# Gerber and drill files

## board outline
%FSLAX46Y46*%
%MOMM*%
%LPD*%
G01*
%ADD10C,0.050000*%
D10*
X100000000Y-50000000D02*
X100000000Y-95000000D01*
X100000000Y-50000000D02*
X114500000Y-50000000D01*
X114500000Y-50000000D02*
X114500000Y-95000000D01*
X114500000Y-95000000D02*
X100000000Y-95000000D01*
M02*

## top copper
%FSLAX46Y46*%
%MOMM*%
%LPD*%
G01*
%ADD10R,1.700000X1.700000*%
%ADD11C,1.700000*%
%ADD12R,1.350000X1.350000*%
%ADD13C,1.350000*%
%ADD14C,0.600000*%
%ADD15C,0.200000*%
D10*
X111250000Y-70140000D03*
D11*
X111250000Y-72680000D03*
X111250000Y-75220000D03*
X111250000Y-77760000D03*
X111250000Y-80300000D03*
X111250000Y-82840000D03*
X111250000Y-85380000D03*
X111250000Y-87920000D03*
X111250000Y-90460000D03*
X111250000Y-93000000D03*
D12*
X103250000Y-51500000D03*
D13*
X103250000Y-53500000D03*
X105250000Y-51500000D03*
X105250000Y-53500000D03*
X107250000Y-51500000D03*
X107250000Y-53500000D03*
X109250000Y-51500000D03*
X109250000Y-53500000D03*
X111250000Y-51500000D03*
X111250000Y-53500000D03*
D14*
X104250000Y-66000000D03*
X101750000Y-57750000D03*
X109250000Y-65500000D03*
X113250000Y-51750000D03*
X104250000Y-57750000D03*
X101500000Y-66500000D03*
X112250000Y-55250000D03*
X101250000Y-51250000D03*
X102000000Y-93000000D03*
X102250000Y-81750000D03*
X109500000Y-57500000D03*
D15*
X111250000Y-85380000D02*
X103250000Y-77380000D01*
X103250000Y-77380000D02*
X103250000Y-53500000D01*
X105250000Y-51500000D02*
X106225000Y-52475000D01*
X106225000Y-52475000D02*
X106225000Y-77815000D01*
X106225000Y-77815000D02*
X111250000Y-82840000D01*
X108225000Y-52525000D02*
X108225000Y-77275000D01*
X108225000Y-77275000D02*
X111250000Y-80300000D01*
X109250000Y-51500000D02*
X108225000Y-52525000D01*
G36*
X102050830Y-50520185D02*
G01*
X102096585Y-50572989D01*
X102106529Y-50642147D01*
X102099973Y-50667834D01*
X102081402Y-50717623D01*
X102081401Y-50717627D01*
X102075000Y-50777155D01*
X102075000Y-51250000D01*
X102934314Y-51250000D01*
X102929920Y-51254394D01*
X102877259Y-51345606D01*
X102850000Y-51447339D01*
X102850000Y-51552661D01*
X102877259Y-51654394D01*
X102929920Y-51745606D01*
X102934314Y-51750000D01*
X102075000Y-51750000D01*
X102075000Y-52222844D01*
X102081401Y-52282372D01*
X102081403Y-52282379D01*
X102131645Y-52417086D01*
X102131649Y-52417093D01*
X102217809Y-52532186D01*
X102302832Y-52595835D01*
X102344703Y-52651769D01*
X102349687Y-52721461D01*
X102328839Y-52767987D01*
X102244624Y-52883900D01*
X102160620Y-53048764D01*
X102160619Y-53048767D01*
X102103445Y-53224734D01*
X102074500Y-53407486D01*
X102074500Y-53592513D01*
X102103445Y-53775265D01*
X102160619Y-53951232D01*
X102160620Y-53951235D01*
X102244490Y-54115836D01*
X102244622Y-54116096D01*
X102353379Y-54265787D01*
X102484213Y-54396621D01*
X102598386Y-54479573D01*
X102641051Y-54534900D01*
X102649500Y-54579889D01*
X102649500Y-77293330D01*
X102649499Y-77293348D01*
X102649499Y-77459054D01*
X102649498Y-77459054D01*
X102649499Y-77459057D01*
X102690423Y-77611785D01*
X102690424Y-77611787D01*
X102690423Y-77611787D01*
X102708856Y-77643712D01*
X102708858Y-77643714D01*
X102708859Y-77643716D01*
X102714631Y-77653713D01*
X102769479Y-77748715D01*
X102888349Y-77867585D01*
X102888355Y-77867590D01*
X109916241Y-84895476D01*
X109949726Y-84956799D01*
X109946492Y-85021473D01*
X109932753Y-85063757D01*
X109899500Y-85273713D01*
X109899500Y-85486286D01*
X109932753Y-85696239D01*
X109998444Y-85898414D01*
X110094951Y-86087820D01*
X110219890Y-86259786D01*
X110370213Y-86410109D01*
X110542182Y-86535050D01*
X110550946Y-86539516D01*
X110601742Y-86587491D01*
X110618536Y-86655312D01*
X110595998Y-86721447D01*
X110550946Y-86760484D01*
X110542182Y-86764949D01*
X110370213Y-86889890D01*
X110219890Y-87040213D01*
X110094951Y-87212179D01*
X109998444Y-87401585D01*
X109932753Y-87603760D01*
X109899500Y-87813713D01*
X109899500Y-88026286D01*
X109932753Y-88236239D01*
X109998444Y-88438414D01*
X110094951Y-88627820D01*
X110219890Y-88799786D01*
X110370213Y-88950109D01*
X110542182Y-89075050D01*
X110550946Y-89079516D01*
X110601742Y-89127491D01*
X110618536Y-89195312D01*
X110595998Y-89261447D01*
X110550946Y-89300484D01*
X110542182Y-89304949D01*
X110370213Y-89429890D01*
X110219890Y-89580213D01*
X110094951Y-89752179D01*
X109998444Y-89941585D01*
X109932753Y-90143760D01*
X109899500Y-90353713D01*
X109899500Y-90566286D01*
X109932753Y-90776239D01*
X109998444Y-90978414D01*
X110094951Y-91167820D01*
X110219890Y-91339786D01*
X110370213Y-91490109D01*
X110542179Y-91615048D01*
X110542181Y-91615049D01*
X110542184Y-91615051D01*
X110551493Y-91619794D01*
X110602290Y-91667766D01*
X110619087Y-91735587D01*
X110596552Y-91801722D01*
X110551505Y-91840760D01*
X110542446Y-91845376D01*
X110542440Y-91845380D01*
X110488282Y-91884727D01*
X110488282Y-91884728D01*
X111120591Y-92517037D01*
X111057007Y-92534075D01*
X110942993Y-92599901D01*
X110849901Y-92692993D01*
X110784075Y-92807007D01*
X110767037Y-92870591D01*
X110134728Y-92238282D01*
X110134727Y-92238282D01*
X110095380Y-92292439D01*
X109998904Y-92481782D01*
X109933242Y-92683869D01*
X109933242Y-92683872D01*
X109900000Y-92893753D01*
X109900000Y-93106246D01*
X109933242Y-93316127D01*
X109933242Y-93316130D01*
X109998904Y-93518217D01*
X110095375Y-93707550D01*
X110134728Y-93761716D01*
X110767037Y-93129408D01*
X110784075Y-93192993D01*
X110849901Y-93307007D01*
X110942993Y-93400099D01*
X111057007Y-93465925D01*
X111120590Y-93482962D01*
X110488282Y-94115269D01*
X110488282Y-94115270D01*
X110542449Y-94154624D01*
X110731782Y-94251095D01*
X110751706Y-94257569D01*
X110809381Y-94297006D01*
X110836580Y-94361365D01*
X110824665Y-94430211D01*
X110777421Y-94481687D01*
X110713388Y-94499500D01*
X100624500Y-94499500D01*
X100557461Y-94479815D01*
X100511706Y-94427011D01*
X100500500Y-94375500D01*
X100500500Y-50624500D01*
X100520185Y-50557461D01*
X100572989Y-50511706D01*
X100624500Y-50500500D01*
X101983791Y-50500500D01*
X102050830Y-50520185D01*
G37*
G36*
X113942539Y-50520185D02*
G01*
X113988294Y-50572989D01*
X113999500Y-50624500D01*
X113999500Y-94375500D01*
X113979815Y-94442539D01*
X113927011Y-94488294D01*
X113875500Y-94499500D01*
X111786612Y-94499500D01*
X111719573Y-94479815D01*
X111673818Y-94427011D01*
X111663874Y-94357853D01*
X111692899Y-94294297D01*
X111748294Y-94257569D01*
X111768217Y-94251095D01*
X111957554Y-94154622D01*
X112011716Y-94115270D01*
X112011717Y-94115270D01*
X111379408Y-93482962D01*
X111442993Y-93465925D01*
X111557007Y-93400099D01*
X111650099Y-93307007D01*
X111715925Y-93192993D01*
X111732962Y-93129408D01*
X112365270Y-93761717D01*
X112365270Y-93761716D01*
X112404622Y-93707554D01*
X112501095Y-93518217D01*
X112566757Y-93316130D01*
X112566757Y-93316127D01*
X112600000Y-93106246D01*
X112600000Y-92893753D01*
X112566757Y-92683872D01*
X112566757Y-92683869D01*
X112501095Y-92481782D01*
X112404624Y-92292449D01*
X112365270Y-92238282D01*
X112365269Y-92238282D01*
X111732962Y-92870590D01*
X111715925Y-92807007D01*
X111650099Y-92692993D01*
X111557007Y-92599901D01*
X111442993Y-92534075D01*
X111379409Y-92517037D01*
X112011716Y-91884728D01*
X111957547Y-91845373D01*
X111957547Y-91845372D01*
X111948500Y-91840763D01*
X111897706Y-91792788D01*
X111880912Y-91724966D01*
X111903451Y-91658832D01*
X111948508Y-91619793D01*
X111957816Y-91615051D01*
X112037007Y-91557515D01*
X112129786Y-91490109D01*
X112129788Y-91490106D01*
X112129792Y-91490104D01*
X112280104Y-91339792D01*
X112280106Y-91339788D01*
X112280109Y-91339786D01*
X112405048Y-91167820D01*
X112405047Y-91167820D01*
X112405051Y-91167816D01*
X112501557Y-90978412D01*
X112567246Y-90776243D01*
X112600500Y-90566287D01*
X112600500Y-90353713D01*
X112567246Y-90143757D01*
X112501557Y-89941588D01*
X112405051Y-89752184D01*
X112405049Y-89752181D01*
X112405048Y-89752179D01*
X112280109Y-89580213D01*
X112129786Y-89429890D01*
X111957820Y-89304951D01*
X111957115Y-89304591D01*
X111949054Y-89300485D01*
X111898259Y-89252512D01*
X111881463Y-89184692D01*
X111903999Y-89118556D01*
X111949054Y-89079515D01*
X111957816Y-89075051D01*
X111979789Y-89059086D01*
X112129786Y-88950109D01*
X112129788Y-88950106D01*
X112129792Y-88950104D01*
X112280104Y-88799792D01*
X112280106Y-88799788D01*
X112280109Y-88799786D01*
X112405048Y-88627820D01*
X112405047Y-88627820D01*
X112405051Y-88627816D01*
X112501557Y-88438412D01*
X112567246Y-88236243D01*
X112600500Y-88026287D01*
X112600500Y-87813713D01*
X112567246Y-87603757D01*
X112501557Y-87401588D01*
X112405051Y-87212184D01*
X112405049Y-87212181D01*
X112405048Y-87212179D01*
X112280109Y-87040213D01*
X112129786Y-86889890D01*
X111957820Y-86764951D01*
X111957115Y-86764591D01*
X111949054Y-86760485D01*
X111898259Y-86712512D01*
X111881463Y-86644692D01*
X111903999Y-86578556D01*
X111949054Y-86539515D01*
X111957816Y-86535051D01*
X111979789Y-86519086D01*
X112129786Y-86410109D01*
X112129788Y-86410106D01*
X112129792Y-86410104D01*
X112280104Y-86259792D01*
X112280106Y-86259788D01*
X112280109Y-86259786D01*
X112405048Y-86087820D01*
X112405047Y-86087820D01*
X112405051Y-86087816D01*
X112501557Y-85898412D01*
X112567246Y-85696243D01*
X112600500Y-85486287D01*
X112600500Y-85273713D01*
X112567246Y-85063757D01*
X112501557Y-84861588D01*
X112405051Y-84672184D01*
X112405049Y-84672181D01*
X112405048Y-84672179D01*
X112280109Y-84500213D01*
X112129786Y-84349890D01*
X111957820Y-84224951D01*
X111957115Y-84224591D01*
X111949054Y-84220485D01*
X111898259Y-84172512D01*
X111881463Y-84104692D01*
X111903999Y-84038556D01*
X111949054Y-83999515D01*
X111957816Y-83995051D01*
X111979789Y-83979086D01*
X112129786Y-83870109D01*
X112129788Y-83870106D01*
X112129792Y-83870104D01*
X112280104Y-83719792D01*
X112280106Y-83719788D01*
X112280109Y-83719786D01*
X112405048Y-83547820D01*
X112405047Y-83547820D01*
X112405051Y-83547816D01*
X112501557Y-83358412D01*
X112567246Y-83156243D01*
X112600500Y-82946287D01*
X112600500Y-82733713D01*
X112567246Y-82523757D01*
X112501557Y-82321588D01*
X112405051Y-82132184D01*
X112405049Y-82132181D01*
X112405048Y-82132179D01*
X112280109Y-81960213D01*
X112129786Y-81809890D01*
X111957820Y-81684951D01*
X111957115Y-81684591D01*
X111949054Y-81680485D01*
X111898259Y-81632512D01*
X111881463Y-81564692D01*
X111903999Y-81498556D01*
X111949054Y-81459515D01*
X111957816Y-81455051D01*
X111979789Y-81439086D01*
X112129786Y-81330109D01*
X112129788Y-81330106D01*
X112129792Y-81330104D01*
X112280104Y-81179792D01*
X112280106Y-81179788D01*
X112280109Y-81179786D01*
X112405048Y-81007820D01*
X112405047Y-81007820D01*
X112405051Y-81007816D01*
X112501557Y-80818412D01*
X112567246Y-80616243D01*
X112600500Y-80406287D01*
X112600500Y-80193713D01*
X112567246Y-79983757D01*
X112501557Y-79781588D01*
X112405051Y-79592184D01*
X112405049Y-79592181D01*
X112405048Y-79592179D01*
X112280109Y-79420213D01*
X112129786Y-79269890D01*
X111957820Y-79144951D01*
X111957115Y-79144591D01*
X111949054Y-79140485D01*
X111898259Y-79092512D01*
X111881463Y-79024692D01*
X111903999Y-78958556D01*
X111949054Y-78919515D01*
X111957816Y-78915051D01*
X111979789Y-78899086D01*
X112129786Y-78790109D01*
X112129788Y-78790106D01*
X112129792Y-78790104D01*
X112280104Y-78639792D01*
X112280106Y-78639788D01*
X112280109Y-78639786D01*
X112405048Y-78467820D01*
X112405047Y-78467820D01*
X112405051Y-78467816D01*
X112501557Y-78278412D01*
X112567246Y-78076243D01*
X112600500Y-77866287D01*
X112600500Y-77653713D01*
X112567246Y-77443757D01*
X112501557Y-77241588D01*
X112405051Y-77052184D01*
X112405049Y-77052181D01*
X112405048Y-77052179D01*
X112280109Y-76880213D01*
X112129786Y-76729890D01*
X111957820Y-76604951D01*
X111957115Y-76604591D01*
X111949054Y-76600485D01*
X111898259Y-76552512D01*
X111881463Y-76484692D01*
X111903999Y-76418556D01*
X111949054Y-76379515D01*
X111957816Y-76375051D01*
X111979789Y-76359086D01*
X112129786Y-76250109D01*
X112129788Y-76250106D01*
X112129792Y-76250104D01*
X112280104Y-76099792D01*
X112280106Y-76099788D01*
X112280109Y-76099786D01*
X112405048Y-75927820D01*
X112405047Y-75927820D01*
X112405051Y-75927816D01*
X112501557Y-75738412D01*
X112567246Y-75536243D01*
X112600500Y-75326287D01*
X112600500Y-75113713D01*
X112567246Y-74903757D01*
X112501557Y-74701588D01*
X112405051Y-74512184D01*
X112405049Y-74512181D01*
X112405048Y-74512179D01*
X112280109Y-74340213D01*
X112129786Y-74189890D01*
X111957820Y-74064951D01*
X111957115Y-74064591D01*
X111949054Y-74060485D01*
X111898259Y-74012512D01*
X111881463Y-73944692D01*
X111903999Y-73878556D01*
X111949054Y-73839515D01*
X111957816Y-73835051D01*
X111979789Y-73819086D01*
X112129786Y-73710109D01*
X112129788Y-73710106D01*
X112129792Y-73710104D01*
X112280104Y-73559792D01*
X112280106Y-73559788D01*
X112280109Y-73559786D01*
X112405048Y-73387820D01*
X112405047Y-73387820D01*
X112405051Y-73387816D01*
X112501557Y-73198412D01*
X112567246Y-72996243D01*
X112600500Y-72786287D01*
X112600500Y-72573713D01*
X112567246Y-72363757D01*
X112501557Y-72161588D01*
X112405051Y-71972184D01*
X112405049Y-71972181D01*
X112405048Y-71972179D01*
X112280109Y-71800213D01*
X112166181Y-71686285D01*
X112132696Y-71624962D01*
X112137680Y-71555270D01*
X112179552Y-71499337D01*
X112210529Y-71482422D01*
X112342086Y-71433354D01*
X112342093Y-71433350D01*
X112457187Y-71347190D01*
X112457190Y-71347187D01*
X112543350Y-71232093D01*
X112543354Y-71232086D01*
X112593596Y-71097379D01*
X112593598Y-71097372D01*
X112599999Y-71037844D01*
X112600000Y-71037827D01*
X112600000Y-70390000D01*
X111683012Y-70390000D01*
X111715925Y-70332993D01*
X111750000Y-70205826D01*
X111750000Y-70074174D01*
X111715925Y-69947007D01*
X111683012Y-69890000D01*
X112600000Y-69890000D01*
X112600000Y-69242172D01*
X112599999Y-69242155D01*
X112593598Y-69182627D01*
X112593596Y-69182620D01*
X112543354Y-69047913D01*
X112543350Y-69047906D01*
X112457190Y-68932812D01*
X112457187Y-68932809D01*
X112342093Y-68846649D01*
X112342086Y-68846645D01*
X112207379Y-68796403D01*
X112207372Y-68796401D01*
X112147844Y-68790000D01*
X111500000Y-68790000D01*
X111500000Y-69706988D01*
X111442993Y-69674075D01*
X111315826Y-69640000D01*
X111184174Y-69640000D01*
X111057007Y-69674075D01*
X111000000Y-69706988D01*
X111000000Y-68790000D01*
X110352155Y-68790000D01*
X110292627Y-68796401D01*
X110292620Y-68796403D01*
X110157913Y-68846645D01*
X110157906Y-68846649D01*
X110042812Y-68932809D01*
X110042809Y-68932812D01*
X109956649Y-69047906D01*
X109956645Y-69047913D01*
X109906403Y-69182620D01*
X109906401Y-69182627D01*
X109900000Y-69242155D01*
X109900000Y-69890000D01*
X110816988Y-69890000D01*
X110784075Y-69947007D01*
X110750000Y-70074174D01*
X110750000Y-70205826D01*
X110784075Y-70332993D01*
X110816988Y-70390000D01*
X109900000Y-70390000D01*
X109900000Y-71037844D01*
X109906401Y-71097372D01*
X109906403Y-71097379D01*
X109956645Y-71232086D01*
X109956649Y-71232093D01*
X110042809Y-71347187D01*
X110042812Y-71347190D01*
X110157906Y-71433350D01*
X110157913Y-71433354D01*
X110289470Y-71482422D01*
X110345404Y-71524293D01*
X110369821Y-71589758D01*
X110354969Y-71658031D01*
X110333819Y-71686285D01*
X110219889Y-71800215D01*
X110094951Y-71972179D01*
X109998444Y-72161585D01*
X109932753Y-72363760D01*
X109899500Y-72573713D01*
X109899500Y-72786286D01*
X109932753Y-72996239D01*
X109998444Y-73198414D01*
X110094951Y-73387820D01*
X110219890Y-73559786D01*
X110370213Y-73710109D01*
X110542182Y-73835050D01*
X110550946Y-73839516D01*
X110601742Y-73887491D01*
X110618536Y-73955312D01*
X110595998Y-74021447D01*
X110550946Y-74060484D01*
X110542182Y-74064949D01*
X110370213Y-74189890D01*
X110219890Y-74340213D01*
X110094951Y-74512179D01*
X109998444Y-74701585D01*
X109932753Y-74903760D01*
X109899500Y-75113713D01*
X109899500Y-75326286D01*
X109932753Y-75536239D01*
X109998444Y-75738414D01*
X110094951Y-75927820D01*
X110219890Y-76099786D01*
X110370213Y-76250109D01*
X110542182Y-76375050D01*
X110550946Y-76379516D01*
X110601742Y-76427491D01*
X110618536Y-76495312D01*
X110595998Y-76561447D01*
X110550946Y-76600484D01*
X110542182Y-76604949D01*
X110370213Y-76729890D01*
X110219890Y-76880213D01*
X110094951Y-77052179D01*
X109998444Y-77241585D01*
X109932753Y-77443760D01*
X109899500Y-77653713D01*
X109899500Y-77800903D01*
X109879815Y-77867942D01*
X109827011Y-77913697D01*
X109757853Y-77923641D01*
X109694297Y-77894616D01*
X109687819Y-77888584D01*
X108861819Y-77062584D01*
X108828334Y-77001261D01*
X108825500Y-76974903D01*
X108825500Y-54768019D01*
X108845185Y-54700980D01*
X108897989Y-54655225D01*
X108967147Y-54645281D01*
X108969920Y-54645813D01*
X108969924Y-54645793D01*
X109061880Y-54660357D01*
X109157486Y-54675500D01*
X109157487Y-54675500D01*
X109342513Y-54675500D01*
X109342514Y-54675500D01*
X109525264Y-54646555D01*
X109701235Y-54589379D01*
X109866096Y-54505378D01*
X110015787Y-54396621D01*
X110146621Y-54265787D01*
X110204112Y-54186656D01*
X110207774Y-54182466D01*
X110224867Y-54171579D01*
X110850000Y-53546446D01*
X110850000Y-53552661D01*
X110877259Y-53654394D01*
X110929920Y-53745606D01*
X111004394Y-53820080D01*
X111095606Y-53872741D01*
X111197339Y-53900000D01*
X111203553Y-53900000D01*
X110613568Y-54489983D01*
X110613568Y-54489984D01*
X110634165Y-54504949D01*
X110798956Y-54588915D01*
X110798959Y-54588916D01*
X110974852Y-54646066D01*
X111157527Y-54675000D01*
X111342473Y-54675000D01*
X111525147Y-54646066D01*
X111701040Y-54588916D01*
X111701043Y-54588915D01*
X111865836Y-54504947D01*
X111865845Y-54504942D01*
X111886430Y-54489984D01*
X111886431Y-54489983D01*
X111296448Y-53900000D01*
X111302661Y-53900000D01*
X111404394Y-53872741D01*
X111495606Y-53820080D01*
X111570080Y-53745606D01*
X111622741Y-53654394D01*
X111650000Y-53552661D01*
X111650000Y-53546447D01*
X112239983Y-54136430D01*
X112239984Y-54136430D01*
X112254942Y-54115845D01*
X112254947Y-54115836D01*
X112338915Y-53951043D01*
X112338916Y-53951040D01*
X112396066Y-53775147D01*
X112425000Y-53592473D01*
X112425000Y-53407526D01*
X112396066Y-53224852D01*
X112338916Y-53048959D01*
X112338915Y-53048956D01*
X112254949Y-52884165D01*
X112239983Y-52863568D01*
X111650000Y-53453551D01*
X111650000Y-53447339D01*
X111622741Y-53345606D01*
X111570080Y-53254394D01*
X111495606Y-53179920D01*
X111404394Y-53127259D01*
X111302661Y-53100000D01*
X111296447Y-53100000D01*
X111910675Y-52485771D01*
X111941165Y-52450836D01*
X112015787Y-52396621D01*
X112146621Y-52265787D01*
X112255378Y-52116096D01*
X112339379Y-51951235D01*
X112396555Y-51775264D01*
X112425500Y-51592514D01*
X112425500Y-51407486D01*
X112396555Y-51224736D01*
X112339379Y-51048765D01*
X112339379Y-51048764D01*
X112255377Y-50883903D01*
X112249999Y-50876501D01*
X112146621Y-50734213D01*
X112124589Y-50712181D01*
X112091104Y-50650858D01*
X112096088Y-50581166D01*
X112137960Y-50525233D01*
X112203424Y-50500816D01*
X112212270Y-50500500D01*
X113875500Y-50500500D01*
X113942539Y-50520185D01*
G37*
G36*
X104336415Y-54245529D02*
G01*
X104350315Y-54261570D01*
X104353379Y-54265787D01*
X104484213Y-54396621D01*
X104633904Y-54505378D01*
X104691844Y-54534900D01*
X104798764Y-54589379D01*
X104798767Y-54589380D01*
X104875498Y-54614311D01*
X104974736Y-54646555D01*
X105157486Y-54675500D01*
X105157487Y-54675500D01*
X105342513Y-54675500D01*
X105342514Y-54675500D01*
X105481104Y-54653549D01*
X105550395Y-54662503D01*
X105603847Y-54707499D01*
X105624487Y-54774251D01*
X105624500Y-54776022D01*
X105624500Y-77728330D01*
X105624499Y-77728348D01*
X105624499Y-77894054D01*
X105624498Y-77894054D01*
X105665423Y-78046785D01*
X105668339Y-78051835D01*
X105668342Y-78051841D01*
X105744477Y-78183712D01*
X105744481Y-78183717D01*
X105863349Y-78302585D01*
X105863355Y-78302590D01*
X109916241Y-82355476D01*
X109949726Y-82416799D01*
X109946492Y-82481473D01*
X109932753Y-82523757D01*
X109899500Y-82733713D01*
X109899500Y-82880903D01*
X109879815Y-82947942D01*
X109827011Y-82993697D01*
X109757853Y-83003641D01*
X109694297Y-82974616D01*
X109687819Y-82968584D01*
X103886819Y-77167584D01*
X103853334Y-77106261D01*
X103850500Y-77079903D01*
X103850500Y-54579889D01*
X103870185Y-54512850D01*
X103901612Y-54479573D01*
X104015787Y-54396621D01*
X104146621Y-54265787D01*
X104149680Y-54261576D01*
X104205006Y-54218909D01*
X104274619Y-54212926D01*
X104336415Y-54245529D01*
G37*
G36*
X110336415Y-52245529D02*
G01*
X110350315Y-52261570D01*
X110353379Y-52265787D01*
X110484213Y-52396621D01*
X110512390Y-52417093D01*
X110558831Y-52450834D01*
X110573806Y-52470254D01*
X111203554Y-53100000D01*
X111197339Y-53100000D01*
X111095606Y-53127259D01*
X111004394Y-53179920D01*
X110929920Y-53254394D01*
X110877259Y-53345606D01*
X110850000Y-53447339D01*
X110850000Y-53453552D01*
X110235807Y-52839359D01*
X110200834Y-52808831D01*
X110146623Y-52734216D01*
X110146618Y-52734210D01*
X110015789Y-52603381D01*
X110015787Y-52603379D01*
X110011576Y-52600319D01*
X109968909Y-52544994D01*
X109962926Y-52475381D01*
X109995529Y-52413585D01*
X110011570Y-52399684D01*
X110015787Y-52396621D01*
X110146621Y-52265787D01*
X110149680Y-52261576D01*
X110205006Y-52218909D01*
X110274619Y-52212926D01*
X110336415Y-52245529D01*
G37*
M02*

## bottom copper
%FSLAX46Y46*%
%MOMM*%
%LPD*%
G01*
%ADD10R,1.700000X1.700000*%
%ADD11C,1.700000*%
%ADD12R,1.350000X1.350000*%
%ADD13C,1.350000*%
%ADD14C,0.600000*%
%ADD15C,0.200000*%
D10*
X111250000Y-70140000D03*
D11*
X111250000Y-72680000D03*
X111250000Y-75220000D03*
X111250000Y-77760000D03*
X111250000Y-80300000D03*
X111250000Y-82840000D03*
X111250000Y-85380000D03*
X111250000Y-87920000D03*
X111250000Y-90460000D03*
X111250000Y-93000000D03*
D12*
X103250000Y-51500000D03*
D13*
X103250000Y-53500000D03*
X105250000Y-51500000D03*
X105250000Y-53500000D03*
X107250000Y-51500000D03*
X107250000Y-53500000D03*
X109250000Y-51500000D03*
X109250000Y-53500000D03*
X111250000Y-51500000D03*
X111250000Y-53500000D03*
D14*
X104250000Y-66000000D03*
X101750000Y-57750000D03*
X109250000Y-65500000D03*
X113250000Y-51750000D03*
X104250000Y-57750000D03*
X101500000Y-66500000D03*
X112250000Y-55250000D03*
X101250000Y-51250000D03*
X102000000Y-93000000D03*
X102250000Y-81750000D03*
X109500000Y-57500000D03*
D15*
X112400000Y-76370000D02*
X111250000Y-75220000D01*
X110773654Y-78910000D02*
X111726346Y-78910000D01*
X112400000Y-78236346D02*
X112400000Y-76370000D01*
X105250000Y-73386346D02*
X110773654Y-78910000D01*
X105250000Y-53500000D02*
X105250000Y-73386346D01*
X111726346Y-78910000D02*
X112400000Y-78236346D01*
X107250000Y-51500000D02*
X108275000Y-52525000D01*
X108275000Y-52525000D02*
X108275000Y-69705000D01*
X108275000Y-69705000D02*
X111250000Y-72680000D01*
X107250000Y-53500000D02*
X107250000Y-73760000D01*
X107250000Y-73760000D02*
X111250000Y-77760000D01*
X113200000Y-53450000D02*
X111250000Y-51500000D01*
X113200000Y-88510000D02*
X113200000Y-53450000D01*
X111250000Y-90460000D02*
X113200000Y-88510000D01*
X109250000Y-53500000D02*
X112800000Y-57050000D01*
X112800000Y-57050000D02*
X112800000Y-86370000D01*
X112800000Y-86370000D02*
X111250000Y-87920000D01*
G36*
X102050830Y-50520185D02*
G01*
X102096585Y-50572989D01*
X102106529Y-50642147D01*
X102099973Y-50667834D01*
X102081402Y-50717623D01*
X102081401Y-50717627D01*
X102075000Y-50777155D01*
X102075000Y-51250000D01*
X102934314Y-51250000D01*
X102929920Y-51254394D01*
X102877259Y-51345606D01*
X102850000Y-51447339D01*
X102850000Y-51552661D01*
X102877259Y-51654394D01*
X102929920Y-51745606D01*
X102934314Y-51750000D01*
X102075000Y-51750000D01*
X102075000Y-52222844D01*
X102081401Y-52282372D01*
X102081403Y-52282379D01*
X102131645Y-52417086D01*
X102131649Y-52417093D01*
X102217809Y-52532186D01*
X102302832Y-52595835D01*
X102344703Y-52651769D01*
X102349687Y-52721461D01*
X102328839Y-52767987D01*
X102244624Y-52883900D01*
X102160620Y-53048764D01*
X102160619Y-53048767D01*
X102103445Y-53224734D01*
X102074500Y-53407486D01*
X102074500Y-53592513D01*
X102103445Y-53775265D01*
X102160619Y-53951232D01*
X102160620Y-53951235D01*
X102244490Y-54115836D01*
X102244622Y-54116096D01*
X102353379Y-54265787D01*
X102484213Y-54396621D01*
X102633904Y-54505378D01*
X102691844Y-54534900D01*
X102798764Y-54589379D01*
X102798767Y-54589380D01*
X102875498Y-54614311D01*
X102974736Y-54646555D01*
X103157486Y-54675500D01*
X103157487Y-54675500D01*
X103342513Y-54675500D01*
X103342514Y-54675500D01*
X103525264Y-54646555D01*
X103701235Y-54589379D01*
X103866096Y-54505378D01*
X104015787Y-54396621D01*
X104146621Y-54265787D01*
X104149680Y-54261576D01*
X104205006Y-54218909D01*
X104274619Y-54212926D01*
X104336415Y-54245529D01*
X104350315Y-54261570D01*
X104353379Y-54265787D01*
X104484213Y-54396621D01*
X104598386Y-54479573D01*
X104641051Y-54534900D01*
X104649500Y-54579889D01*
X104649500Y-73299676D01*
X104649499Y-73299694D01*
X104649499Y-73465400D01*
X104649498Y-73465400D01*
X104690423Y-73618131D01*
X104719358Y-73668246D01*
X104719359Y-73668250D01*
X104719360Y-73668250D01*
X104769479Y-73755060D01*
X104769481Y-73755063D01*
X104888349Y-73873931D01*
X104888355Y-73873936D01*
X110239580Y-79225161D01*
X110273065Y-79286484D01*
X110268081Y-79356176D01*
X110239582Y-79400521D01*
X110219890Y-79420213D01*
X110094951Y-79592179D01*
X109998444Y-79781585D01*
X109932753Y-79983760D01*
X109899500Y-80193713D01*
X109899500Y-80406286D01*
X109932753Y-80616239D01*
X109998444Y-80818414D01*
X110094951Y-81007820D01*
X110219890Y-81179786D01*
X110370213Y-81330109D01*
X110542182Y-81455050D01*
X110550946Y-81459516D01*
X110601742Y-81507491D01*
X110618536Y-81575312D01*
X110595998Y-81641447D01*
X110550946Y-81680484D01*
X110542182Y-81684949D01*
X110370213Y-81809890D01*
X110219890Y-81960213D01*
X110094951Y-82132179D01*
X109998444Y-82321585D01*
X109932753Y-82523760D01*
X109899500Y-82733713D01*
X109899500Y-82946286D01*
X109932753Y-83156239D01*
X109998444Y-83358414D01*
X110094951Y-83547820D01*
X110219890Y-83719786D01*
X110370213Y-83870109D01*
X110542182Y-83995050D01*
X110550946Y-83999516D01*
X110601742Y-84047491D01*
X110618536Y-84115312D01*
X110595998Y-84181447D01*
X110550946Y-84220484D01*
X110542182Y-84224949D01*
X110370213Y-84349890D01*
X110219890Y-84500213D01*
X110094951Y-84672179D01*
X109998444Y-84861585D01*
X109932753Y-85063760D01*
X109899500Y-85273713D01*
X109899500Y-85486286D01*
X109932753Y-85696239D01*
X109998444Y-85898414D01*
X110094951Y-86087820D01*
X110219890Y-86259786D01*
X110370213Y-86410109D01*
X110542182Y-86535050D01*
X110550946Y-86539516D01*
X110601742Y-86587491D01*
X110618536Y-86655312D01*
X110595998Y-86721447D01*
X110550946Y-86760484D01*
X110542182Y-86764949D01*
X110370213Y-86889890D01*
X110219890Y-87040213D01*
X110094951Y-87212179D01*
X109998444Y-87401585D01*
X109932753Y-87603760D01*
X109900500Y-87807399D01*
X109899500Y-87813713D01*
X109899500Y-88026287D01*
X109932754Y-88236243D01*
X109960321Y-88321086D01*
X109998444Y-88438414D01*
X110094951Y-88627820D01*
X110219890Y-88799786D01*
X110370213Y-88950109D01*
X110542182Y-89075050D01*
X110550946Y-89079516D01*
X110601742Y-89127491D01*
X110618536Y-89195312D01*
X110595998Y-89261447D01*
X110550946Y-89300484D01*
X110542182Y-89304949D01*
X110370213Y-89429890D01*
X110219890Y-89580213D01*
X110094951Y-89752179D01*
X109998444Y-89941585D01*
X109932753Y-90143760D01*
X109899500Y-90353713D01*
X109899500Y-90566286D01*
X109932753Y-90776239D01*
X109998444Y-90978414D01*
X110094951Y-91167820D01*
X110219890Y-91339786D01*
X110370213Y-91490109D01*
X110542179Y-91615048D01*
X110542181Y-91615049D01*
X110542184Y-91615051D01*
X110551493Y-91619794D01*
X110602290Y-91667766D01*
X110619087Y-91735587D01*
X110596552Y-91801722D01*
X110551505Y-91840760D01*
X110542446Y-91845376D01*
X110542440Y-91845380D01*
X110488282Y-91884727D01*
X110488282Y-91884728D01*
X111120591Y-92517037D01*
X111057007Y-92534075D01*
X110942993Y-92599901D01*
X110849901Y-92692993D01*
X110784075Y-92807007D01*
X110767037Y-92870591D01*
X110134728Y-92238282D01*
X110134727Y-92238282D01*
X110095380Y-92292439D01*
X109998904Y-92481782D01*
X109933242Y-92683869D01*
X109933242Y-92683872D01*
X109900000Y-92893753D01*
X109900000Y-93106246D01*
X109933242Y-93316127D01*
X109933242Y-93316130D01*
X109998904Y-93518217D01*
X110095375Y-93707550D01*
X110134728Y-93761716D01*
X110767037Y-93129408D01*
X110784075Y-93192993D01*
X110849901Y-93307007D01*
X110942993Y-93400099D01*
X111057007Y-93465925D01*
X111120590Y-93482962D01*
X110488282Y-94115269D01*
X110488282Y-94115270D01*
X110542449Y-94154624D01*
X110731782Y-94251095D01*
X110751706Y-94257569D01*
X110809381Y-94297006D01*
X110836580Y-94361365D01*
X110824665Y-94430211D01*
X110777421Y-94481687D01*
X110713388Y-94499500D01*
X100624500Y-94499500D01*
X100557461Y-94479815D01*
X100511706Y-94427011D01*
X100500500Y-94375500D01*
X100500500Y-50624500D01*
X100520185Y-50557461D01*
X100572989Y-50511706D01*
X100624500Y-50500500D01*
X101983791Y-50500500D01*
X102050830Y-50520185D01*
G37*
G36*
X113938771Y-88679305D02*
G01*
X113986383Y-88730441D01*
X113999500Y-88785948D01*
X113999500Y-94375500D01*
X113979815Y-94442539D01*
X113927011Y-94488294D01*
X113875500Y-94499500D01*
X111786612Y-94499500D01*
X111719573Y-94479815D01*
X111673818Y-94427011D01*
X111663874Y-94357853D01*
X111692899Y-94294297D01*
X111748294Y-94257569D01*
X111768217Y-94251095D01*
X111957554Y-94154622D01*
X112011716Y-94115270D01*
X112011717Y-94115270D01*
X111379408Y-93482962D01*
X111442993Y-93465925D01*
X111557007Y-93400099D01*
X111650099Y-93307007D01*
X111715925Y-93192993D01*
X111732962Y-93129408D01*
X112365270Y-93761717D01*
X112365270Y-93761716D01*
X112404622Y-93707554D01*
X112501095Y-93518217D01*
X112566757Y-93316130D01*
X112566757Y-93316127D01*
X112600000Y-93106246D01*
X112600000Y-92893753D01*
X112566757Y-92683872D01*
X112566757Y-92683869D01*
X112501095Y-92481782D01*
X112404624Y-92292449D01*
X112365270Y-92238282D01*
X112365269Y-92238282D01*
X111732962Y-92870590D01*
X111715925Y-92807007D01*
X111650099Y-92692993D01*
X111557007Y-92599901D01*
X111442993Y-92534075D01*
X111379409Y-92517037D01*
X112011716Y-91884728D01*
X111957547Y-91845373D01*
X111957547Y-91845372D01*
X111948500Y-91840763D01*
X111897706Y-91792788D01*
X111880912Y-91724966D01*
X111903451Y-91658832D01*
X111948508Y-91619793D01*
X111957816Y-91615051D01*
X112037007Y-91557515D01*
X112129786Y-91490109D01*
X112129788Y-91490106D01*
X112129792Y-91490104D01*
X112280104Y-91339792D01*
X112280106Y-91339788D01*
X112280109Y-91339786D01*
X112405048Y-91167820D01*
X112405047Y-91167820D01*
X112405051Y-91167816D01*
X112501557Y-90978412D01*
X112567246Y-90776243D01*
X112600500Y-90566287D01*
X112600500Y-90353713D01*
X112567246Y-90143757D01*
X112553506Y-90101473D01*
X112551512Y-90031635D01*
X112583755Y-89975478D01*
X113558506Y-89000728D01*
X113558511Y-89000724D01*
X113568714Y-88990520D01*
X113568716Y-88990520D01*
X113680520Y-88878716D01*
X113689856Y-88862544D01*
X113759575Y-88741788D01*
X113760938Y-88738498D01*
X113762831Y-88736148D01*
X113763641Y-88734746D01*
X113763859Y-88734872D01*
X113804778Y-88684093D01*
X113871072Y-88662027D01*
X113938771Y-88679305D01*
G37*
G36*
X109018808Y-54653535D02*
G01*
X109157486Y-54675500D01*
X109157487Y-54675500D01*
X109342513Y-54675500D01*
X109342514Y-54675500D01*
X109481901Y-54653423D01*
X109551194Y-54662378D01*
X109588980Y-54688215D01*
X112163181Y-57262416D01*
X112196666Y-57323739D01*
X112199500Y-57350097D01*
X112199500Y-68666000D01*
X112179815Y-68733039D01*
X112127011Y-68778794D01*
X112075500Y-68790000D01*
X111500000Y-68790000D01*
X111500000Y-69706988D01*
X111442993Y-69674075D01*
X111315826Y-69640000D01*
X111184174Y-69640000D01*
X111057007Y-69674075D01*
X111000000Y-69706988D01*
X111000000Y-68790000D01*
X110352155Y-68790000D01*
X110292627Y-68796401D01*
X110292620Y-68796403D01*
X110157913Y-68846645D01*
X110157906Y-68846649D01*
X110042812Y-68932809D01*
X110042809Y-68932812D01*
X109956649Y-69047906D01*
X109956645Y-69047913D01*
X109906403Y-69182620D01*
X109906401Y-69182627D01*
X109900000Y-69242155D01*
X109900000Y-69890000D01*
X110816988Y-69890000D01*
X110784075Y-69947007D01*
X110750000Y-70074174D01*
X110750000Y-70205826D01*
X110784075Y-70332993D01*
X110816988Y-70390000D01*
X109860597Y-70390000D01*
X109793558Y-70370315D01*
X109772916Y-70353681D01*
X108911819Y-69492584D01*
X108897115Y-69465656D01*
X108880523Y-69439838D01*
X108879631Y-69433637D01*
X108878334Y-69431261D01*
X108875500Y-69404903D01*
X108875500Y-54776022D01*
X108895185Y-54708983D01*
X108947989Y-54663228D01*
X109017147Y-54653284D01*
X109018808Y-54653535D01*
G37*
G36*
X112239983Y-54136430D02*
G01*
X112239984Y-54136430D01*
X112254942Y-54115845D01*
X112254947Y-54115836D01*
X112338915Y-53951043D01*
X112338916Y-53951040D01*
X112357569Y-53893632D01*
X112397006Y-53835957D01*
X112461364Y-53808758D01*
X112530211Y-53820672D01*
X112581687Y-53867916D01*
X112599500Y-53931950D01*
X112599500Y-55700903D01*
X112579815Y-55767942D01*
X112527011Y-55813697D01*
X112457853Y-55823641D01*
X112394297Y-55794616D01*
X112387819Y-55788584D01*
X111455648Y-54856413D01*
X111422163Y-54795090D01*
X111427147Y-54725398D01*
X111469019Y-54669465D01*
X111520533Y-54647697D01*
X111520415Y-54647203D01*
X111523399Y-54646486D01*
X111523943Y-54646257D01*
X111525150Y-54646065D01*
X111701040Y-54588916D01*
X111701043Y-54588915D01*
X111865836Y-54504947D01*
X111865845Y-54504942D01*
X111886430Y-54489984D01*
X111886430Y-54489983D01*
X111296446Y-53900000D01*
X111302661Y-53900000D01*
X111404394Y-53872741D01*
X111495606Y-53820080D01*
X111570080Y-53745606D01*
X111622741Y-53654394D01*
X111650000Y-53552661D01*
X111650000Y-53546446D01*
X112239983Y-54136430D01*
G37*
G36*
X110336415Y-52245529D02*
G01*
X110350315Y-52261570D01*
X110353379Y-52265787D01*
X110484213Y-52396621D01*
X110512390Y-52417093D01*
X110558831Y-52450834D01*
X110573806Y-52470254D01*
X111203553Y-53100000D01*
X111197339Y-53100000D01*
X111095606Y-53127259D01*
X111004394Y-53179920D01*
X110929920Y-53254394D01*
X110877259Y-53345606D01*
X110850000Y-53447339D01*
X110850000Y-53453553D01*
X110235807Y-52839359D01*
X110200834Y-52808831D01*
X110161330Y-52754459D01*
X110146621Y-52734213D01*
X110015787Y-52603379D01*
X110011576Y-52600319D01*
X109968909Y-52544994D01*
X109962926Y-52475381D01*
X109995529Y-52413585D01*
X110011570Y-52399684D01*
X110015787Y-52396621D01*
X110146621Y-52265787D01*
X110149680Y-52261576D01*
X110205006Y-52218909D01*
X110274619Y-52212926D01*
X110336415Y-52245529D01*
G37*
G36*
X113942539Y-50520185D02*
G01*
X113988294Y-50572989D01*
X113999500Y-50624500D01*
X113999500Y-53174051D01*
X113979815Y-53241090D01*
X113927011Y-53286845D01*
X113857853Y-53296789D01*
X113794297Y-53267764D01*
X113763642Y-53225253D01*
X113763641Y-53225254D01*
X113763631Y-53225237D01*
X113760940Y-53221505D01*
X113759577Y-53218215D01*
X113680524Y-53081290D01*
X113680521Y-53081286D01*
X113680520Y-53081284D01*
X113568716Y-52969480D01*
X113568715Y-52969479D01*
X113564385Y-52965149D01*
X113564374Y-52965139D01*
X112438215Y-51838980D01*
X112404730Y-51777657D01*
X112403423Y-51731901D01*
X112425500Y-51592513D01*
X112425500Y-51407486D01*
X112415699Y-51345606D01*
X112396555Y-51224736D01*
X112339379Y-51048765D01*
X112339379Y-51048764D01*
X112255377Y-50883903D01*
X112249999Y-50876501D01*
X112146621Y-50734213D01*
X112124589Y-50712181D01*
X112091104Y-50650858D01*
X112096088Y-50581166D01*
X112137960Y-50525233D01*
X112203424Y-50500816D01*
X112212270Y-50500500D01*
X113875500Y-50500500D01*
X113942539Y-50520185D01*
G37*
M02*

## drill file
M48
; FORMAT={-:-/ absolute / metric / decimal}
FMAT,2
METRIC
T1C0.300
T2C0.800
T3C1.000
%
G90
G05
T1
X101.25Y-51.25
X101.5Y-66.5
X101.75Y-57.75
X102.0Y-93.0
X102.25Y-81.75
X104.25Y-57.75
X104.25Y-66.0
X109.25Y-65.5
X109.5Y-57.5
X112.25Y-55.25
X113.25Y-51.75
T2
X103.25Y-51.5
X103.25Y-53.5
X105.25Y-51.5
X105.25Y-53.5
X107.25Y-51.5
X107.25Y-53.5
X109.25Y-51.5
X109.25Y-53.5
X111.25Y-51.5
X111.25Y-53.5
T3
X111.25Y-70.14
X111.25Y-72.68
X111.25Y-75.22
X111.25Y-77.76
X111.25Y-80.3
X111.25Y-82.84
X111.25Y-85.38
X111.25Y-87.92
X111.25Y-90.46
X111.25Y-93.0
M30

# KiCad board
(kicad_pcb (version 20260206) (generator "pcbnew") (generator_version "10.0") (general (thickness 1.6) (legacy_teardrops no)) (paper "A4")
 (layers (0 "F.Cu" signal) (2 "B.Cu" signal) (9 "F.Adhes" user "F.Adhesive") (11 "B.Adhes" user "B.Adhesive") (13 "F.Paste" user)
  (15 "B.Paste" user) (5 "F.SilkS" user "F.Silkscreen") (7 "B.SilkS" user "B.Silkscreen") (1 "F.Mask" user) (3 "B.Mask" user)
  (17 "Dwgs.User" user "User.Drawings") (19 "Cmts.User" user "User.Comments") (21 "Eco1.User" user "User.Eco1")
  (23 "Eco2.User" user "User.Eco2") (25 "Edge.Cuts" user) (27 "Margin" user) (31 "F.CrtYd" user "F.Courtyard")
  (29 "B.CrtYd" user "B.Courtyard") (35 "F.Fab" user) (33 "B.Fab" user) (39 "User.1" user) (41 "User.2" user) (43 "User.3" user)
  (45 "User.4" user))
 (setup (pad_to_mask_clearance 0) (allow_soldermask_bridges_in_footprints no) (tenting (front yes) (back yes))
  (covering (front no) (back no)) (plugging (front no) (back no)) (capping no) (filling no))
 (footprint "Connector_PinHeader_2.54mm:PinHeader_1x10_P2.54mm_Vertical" (layer "F.Cu") (at 111.25 70.14)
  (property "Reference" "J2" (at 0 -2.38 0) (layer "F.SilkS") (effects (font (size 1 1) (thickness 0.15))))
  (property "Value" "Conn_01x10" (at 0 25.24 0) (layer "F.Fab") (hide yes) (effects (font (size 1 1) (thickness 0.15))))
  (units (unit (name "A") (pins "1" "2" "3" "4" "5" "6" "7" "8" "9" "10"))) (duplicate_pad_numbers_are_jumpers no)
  (pad "1" thru_hole rect (at 0 0) (size 1.7 1.7) (drill 1) (layers "*.Cu" "*.Mask") (remove_unused_layers no) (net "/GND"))
  (pad "2" thru_hole circle (at 0 2.54) (size 1.7 1.7) (drill 1) (layers "*.Cu" "*.Mask") (remove_unused_layers no) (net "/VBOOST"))
  (pad "3" thru_hole circle (at 0 5.08) (size 1.7 1.7) (drill 1) (layers "*.Cu" "*.Mask") (remove_unused_layers no) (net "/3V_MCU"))
  (pad "4" thru_hole circle (at 0 7.62) (size 1.7 1.7) (drill 1) (layers "*.Cu" "*.Mask") (remove_unused_layers no) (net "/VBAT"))
  (pad "5" thru_hole circle (at 0 10.16) (size 1.7 1.7) (drill 1) (layers "*.Cu" "*.Mask") (remove_unused_layers no) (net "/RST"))
  (pad "6" thru_hole circle (at 0 12.7) (size 1.7 1.7) (drill 1) (layers "*.Cu" "*.Mask") (remove_unused_layers no) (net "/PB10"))
  (pad "7" thru_hole circle (at 0 15.24) (size 1.7 1.7) (drill 1) (layers "*.Cu" "*.Mask") (remove_unused_layers no) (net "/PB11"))
  (pad "8" thru_hole circle (at 0 17.78) (size 1.7 1.7) (drill 1) (layers "*.Cu" "*.Mask") (remove_unused_layers no) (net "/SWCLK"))
  (pad "9" thru_hole circle (at 0 20.32) (size 1.7 1.7) (drill 1) (layers "*.Cu" "*.Mask") (remove_unused_layers no) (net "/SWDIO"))
  (pad "10" thru_hole circle (at 0 22.86) (size 1.7 1.7) (drill 1) (layers "*.Cu" "*.Mask") (remove_unused_layers no) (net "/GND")))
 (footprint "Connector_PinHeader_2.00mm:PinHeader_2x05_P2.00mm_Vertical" (layer "B.Cu") (at 103.25 51.5 -90)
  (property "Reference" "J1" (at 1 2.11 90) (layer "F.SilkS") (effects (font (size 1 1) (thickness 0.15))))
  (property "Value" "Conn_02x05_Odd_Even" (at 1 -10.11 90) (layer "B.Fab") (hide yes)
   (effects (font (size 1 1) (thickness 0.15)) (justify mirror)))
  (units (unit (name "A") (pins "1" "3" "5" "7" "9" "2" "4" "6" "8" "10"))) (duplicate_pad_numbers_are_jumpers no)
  (pad "1" thru_hole rect (at 0 0 270) (size 1.35 1.35) (drill 0.8) (layers "*.Cu" "*.Mask") (remove_unused_layers no) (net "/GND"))
  (pad "2" thru_hole circle (at 2 0 270) (size 1.35 1.35) (drill 0.8) (layers "*.Cu" "*.Mask") (remove_unused_layers no) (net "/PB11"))
  (pad "3" thru_hole circle (at 0 -2 270) (size 1.35 1.35) (drill 0.8) (layers "*.Cu" "*.Mask") (remove_unused_layers no) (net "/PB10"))
  (pad "4" thru_hole circle (at 2 -2 270) (size 1.35 1.35) (drill 0.8) (layers "*.Cu" "*.Mask") (remove_unused_layers no) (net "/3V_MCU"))
  (pad "5" thru_hole circle (at 0 -4 270) (size 1.35 1.35) (drill 0.8) (layers "*.Cu" "*.Mask") (remove_unused_layers no) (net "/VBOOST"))
  (pad "6" thru_hole circle (at 2 -4 270) (size 1.35 1.35) (drill 0.8) (layers "*.Cu" "*.Mask") (remove_unused_layers no) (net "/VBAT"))
  (pad "7" thru_hole circle (at 0 -6 270) (size 1.35 1.35) (drill 0.8) (layers "*.Cu" "*.Mask") (remove_unused_layers no) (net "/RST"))
  (pad "8" thru_hole circle (at 2 -6 270) (size 1.35 1.35) (drill 0.8) (layers "*.Cu" "*.Mask") (remove_unused_layers no) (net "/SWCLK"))
  (pad "9" thru_hole circle (at 0 -8 270) (size 1.35 1.35) (drill 0.8) (layers "*.Cu" "*.Mask") (remove_unused_layers no) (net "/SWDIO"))
  (pad "10" thru_hole circle (at 2 -8 270) (size 1.35 1.35) (drill 0.8) (layers "*.Cu" "*.Mask") (remove_unused_layers no) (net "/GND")))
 (gr_line (start 100 50) (end 100 95) (stroke (width 0.05) (type default)) (layer "Edge.Cuts"))
 (gr_line (start 100 50) (end 114.5 50) (stroke (width 0.05) (type default)) (layer "Edge.Cuts"))
 (gr_line (start 114.5 50) (end 114.5 95) (stroke (width 0.05) (type default)) (layer "Edge.Cuts"))
 (gr_line (start 114.5 95) (end 100 95) (stroke (width 0.05) (type default)) (layer "Edge.Cuts"))
 (segment (start 112.4 76.37) (end 111.25 75.22) (width 0.2) (layer "B.Cu") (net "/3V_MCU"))
 (segment (start 110.773654 78.91) (end 111.726346 78.91) (width 0.2) (layer "B.Cu") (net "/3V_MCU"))
 (segment (start 112.4 78.236346) (end 112.4 76.37) (width 0.2) (layer "B.Cu") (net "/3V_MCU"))
 (segment (start 105.25 73.386346) (end 110.773654 78.91) (width 0.2) (layer "B.Cu") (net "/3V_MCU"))
 (segment (start 105.25 53.5) (end 105.25 73.386346) (width 0.2) (layer "B.Cu") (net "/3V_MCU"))
 (segment (start 111.726346 78.91) (end 112.4 78.236346) (width 0.2) (layer "B.Cu") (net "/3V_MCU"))
 (segment (start 107.25 51.5) (end 108.275 52.525) (width 0.2) (layer "B.Cu") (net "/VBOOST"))
 (segment (start 108.275 52.525) (end 108.275 69.705) (width 0.2) (layer "B.Cu") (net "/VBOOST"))
 (segment (start 108.275 69.705) (end 111.25 72.68) (width 0.2) (layer "B.Cu") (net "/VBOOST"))
 (via (at 104.25 66) (size 0.6) (drill 0.3) (layers "F.Cu" "B.Cu") (free yes) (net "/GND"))
 (via (at 101.75 57.75) (size 0.6) (drill 0.3) (layers "F.Cu" "B.Cu") (free yes) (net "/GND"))
 (via (at 109.25 65.5) (size 0.6) (drill 0.3) (layers "F.Cu" "B.Cu") (free yes) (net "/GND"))
 (via (at 113.25 51.75) (size 0.6) (drill 0.3) (layers "F.Cu" "B.Cu") (free yes) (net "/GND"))
 (via (at 104.25 57.75) (size 0.6) (drill 0.3) (layers "F.Cu" "B.Cu") (free yes) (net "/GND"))
 (via (at 101.5 66.5) (size 0.6) (drill 0.3) (layers "F.Cu" "B.Cu") (free yes) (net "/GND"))
 (via (at 112.25 55.25) (size 0.6) (drill 0.3) (layers "F.Cu" "B.Cu") (free yes) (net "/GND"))
 (via (at 101.25 51.25) (size 0.6) (drill 0.3) (layers "F.Cu" "B.Cu") (free yes) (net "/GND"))
 (via (at 102 93) (size 0.6) (drill 0.3) (layers "F.Cu" "B.Cu") (free yes) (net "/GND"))
 (via (at 102.25 81.75) (size 0.6) (drill 0.3) (layers "F.Cu" "B.Cu") (free yes) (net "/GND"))
 (via (at 109.5 57.5) (size 0.6) (drill 0.3) (layers "F.Cu" "B.Cu") (free yes) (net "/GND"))
 (segment (start 111.25 85.38) (end 103.25 77.38) (width 0.2) (layer "F.Cu") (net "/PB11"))
 (segment (start 103.25 77.38) (end 103.25 53.5) (width 0.2) (layer "F.Cu") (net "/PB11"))
 (segment (start 105.25 51.5) (end 106.225 52.475) (width 0.2) (layer "F.Cu") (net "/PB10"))
 (segment (start 106.225 52.475) (end 106.225 77.815) (width 0.2) (layer "F.Cu") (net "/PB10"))
 (segment (start 106.225 77.815) (end 111.25 82.84) (width 0.2) (layer "F.Cu") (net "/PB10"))
 (segment (start 107.25 53.5) (end 107.25 73.76) (width 0.2) (layer "B.Cu") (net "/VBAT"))
 (segment (start 107.25 73.76) (end 111.25 77.76) (width 0.2) (layer "B.Cu") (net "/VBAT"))
 (segment (start 113.2 53.45) (end 111.25 51.5) (width 0.2) (layer "B.Cu") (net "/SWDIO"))
 (segment (start 113.2 88.51) (end 113.2 53.45) (width 0.2) (layer "B.Cu") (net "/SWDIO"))
 (segment (start 111.25 90.46) (end 113.2 88.51) (width 0.2) (layer "B.Cu") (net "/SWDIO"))
 (segment (start 108.225 52.525) (end 108.225 77.275) (width 0.2) (layer "F.Cu") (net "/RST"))
 (segment (start 108.225 77.275) (end 111.25 80.3) (width 0.2) (layer "F.Cu") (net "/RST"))
 (segment (start 109.25 51.5) (end 108.225 52.525) (width 0.2) (layer "F.Cu") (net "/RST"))
 (segment (start 109.25 53.5) (end 112.8 57.05) (width 0.2) (layer "B.Cu") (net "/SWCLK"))
 (segment (start 112.8 57.05) (end 112.8 86.37) (width 0.2) (layer "B.Cu") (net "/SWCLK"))
 (segment (start 112.8 86.37) (end 111.25 87.92) (width 0.2) (layer "B.Cu") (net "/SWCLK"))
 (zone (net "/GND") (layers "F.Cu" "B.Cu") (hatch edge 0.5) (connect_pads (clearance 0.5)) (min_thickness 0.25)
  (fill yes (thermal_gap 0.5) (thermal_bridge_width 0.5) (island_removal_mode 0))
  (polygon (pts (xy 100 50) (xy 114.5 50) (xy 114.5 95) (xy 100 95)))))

